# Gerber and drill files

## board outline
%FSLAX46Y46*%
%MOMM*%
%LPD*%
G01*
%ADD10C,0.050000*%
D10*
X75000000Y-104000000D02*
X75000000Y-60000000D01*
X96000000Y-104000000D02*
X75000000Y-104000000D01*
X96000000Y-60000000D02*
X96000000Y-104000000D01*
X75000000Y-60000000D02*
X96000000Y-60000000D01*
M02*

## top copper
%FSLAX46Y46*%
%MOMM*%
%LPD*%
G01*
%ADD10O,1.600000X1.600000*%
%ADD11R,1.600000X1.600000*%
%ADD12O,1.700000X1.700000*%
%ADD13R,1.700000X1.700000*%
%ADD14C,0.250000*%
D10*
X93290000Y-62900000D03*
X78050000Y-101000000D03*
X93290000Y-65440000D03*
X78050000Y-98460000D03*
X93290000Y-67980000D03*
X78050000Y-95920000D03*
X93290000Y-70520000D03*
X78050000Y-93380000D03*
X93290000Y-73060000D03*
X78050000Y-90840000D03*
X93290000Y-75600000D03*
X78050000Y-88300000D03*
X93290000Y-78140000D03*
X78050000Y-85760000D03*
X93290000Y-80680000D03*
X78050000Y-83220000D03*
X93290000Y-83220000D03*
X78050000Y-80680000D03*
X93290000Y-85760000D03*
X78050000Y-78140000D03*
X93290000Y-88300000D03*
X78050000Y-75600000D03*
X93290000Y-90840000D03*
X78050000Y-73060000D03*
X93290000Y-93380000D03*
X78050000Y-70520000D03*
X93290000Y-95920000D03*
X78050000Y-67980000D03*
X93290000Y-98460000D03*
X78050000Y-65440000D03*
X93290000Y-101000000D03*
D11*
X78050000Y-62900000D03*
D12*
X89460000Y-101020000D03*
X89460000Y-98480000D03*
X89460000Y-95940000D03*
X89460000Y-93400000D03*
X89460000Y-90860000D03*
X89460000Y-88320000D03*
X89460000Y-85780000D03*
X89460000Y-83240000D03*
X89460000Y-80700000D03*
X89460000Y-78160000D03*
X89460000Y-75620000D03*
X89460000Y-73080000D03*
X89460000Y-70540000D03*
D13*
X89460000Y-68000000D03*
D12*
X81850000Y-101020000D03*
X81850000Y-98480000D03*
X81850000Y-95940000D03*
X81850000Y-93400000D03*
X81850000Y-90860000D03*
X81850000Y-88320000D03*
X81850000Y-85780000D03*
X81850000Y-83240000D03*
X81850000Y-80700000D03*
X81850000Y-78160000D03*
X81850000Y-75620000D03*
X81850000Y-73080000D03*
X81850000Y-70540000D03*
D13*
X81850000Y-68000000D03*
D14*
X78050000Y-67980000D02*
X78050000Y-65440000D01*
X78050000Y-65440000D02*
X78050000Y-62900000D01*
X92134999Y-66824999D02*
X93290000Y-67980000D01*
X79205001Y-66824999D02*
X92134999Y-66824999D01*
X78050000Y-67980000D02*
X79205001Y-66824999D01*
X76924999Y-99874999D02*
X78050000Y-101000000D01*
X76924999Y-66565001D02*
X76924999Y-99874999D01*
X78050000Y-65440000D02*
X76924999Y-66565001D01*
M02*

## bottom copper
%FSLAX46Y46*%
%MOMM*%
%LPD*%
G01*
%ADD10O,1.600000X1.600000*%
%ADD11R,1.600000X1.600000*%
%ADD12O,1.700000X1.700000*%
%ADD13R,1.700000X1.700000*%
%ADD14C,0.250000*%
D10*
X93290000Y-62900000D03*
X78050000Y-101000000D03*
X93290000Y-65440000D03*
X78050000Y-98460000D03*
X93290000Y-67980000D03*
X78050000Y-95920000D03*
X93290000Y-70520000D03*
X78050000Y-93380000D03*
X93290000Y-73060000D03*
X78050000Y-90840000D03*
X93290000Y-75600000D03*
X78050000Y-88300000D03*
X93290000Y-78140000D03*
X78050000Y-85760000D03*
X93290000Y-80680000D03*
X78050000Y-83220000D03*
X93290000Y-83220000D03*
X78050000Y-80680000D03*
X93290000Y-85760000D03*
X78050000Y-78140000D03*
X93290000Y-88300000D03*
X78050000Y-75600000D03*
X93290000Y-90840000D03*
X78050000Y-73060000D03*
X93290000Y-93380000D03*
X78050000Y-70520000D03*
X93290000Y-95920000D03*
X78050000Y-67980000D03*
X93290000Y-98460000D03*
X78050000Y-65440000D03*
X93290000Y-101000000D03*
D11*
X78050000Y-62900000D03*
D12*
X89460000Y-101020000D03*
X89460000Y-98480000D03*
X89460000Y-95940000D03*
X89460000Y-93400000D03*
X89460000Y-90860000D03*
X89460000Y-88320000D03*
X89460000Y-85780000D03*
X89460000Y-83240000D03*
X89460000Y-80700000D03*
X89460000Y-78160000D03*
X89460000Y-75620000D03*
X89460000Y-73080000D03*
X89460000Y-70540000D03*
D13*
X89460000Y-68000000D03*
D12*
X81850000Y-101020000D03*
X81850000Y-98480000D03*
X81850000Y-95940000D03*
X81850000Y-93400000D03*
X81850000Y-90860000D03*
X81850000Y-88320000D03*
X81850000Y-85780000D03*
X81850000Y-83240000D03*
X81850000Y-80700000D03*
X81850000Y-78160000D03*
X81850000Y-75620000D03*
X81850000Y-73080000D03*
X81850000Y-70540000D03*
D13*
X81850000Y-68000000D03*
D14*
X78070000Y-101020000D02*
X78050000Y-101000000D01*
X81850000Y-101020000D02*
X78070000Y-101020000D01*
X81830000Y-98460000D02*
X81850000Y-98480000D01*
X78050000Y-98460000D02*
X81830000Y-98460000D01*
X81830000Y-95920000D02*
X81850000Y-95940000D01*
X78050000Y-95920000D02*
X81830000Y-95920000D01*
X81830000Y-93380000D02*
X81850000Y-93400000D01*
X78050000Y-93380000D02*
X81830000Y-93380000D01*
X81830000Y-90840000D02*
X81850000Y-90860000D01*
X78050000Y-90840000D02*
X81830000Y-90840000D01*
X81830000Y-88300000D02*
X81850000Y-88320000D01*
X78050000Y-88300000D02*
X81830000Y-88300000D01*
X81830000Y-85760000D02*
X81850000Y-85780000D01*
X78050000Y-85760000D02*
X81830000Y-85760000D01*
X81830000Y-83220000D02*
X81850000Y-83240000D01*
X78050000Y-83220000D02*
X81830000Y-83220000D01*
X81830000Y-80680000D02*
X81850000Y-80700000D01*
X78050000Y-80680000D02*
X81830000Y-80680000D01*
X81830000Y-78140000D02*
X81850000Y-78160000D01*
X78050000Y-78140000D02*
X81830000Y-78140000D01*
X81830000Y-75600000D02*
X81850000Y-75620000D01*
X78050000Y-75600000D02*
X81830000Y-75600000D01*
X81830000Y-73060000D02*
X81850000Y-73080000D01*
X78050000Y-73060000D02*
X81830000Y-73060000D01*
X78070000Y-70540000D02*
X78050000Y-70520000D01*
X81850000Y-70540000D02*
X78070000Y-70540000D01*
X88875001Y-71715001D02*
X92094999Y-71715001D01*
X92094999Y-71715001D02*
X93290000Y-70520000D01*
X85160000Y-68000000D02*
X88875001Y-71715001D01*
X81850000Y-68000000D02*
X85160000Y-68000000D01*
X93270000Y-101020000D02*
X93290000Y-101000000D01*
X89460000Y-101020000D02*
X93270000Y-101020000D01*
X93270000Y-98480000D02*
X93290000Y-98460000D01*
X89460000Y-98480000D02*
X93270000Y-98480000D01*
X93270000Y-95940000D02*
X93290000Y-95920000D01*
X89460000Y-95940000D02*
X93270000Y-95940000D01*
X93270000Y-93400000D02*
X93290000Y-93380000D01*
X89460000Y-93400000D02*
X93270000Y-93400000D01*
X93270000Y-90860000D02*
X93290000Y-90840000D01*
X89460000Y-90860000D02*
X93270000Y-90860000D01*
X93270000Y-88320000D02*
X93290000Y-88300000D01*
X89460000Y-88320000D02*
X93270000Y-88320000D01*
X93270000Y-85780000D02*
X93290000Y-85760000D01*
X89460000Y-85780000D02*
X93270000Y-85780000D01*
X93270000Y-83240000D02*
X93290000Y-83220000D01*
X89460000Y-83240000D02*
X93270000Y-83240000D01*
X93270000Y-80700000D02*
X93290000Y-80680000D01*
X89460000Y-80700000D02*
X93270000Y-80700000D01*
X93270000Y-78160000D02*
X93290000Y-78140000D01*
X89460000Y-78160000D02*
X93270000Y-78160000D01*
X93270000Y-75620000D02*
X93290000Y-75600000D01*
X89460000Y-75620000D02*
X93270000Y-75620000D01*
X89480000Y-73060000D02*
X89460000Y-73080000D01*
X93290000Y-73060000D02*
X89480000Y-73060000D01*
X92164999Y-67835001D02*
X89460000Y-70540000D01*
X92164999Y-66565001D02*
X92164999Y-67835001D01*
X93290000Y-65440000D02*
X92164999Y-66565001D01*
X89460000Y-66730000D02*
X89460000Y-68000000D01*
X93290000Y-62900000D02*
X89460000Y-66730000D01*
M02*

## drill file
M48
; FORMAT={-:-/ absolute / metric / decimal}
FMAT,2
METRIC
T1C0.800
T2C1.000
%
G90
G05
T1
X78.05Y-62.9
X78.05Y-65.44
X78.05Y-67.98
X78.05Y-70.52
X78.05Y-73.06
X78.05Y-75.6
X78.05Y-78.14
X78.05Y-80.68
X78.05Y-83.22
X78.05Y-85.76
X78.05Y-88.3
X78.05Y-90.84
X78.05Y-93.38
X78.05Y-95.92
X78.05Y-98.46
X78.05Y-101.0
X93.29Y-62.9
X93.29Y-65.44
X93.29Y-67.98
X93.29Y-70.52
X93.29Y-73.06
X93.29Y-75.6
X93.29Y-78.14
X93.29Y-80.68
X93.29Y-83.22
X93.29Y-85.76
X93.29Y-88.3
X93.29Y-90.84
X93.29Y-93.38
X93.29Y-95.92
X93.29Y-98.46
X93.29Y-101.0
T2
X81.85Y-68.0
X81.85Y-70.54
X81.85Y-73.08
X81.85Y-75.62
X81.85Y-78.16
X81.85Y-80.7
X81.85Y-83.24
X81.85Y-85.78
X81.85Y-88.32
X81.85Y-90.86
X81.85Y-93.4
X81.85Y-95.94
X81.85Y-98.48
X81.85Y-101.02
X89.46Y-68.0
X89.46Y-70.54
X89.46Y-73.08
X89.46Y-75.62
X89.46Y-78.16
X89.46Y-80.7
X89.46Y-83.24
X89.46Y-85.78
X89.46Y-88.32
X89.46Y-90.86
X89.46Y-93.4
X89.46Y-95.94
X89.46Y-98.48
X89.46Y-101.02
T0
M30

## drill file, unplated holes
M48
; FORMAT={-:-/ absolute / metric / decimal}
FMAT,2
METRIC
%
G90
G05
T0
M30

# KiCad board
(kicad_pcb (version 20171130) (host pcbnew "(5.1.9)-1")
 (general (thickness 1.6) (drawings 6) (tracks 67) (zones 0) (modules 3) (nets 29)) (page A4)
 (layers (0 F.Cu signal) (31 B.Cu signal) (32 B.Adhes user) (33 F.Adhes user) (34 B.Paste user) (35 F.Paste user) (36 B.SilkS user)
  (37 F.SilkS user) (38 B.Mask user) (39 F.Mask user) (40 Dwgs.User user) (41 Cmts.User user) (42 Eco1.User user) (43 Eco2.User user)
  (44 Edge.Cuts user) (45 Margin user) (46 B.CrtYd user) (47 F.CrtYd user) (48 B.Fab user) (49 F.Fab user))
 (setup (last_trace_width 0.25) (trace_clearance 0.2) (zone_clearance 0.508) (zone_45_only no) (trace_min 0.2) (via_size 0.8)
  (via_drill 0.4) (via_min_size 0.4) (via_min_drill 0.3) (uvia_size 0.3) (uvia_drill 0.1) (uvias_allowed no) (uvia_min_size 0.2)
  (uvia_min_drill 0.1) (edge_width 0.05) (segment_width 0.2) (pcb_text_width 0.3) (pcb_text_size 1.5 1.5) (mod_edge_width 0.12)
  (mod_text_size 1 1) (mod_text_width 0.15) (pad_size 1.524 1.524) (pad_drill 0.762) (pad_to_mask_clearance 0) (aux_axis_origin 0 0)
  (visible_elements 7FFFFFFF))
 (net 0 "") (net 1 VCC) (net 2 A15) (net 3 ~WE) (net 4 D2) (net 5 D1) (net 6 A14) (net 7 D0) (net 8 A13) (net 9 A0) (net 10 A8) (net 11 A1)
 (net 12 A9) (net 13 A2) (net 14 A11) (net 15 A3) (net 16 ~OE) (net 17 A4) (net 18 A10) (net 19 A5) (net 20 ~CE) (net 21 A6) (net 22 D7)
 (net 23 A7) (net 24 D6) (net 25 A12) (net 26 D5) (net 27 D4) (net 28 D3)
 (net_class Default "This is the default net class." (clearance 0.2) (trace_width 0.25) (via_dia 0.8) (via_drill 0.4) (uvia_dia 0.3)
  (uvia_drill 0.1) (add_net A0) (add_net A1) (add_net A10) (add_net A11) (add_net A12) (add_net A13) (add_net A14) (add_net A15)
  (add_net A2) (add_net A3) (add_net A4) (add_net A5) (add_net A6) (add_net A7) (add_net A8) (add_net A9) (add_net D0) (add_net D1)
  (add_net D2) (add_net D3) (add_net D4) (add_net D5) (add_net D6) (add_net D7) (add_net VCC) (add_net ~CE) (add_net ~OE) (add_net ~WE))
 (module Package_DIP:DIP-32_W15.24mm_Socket (layer F.Cu) (at 78.05 62.9)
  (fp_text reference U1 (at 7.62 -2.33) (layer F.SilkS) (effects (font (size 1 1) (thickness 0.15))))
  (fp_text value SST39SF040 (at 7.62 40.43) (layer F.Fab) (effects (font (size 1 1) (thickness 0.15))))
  (pad 32 thru_hole oval (at 15.24 0) (size 1.6 1.6) (drill 0.8) (layers *.Cu *.Mask) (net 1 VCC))
  (pad 16 thru_hole oval (at 0 38.1) (size 1.6 1.6) (drill 0.8) (layers *.Cu *.Mask) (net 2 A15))
  (pad 31 thru_hole oval (at 15.24 2.54) (size 1.6 1.6) (drill 0.8) (layers *.Cu *.Mask) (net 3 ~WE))
  (pad 15 thru_hole oval (at 0 35.56) (size 1.6 1.6) (drill 0.8) (layers *.Cu *.Mask) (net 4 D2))
  (pad 30 thru_hole oval (at 15.24 5.08) (size 1.6 1.6) (drill 0.8) (layers *.Cu *.Mask) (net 2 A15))
  (pad 14 thru_hole oval (at 0 33.02) (size 1.6 1.6) (drill 0.8) (layers *.Cu *.Mask) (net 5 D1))
  (pad 29 thru_hole oval (at 15.24 7.62) (size 1.6 1.6) (drill 0.8) (layers *.Cu *.Mask) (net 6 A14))
  (pad 13 thru_hole oval (at 0 30.48) (size 1.6 1.6) (drill 0.8) (layers *.Cu *.Mask) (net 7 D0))
  (pad 28 thru_hole oval (at 15.24 10.16) (size 1.6 1.6) (drill 0.8) (layers *.Cu *.Mask) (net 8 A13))
  (pad 12 thru_hole oval (at 0 27.94) (size 1.6 1.6) (drill 0.8) (layers *.Cu *.Mask) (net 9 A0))
  (pad 27 thru_hole oval (at 15.24 12.7) (size 1.6 1.6) (drill 0.8) (layers *.Cu *.Mask) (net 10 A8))
  (pad 11 thru_hole oval (at 0 25.4) (size 1.6 1.6) (drill 0.8) (layers *.Cu *.Mask) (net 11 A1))
  (pad 26 thru_hole oval (at 15.24 15.24) (size 1.6 1.6) (drill 0.8) (layers *.Cu *.Mask) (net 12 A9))
  (pad 10 thru_hole oval (at 0 22.86) (size 1.6 1.6) (drill 0.8) (layers *.Cu *.Mask) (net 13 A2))
  (pad 25 thru_hole oval (at 15.24 17.78) (size 1.6 1.6) (drill 0.8) (layers *.Cu *.Mask) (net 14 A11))
  (pad 9 thru_hole oval (at 0 20.32) (size 1.6 1.6) (drill 0.8) (layers *.Cu *.Mask) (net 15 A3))
  (pad 24 thru_hole oval (at 15.24 20.32) (size 1.6 1.6) (drill 0.8) (layers *.Cu *.Mask) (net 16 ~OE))
  (pad 8 thru_hole oval (at 0 17.78) (size 1.6 1.6) (drill 0.8) (layers *.Cu *.Mask) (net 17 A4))
  (pad 23 thru_hole oval (at 15.24 22.86) (size 1.6 1.6) (drill 0.8) (layers *.Cu *.Mask) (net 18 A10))
  (pad 7 thru_hole oval (at 0 15.24) (size 1.6 1.6) (drill 0.8) (layers *.Cu *.Mask) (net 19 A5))
  (pad 22 thru_hole oval (at 15.24 25.4) (size 1.6 1.6) (drill 0.8) (layers *.Cu *.Mask) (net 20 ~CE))
  (pad 6 thru_hole oval (at 0 12.7) (size 1.6 1.6) (drill 0.8) (layers *.Cu *.Mask) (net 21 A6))
  (pad 21 thru_hole oval (at 15.24 27.94) (size 1.6 1.6) (drill 0.8) (layers *.Cu *.Mask) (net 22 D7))
  (pad 5 thru_hole oval (at 0 10.16) (size 1.6 1.6) (drill 0.8) (layers *.Cu *.Mask) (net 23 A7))
  (pad 20 thru_hole oval (at 15.24 30.48) (size 1.6 1.6) (drill 0.8) (layers *.Cu *.Mask) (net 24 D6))
  (pad 4 thru_hole oval (at 0 7.62) (size 1.6 1.6) (drill 0.8) (layers *.Cu *.Mask) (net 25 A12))
  (pad 19 thru_hole oval (at 15.24 33.02) (size 1.6 1.6) (drill 0.8) (layers *.Cu *.Mask) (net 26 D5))
  (pad 3 thru_hole oval (at 0 5.08) (size 1.6 1.6) (drill 0.8) (layers *.Cu *.Mask) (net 2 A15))
  (pad 18 thru_hole oval (at 15.24 35.56) (size 1.6 1.6) (drill 0.8) (layers *.Cu *.Mask) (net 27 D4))
  (pad 2 thru_hole oval (at 0 2.54) (size 1.6 1.6) (drill 0.8) (layers *.Cu *.Mask) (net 2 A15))
  (pad 17 thru_hole oval (at 15.24 38.1) (size 1.6 1.6) (drill 0.8) (layers *.Cu *.Mask) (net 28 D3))
  (pad 1 thru_hole rect (at 0 0) (size 1.6 1.6) (drill 0.8) (layers *.Cu *.Mask) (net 2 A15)))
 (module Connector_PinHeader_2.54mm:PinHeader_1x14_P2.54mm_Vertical (layer B.Cu) (at 89.46 68 180)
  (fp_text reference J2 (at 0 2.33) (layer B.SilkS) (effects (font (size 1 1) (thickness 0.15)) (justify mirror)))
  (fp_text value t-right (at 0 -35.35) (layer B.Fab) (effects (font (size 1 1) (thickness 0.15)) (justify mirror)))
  (pad 14 thru_hole oval (at 0 -33.02 180) (size 1.7 1.7) (drill 1) (layers *.Cu *.Mask) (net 28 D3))
  (pad 13 thru_hole oval (at 0 -30.48 180) (size 1.7 1.7) (drill 1) (layers *.Cu *.Mask) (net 27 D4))
  (pad 12 thru_hole oval (at 0 -27.94 180) (size 1.7 1.7) (drill 1) (layers *.Cu *.Mask) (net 26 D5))
  (pad 11 thru_hole oval (at 0 -25.4 180) (size 1.7 1.7) (drill 1) (layers *.Cu *.Mask) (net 24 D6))
  (pad 10 thru_hole oval (at 0 -22.86 180) (size 1.7 1.7) (drill 1) (layers *.Cu *.Mask) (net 22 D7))
  (pad 9 thru_hole oval (at 0 -20.32 180) (size 1.7 1.7) (drill 1) (layers *.Cu *.Mask) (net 20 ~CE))
  (pad 8 thru_hole oval (at 0 -17.78 180) (size 1.7 1.7) (drill 1) (layers *.Cu *.Mask) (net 18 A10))
  (pad 7 thru_hole oval (at 0 -15.24 180) (size 1.7 1.7) (drill 1) (layers *.Cu *.Mask) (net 16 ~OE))
  (pad 6 thru_hole oval (at 0 -12.7 180) (size 1.7 1.7) (drill 1) (layers *.Cu *.Mask) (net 14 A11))
  (pad 5 thru_hole oval (at 0 -10.16 180) (size 1.7 1.7) (drill 1) (layers *.Cu *.Mask) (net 12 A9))
  (pad 4 thru_hole oval (at 0 -7.62 180) (size 1.7 1.7) (drill 1) (layers *.Cu *.Mask) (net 10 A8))
  (pad 3 thru_hole oval (at 0 -5.08 180) (size 1.7 1.7) (drill 1) (layers *.Cu *.Mask) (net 8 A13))
  (pad 2 thru_hole oval (at 0 -2.54 180) (size 1.7 1.7) (drill 1) (layers *.Cu *.Mask) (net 3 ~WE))
  (pad 1 thru_hole rect (at 0 0 180) (size 1.7 1.7) (drill 1) (layers *.Cu *.Mask) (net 1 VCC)))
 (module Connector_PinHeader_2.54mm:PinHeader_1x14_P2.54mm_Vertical (layer B.Cu) (at 81.85 68 180)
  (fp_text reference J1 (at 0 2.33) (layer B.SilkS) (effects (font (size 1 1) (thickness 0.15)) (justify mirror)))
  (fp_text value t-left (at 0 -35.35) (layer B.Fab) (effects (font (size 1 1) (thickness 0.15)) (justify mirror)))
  (pad 14 thru_hole oval (at 0 -33.02 180) (size 1.7 1.7) (drill 1) (layers *.Cu *.Mask) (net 2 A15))
  (pad 13 thru_hole oval (at 0 -30.48 180) (size 1.7 1.7) (drill 1) (layers *.Cu *.Mask) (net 4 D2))
  (pad 12 thru_hole oval (at 0 -27.94 180) (size 1.7 1.7) (drill 1) (layers *.Cu *.Mask) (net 5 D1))
  (pad 11 thru_hole oval (at 0 -25.4 180) (size 1.7 1.7) (drill 1) (layers *.Cu *.Mask) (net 7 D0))
  (pad 10 thru_hole oval (at 0 -22.86 180) (size 1.7 1.7) (drill 1) (layers *.Cu *.Mask) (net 9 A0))
  (pad 9 thru_hole oval (at 0 -20.32 180) (size 1.7 1.7) (drill 1) (layers *.Cu *.Mask) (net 11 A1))
  (pad 8 thru_hole oval (at 0 -17.78 180) (size 1.7 1.7) (drill 1) (layers *.Cu *.Mask) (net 13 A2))
  (pad 7 thru_hole oval (at 0 -15.24 180) (size 1.7 1.7) (drill 1) (layers *.Cu *.Mask) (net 15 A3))
  (pad 6 thru_hole oval (at 0 -12.7 180) (size 1.7 1.7) (drill 1) (layers *.Cu *.Mask) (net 17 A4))
  (pad 5 thru_hole oval (at 0 -10.16 180) (size 1.7 1.7) (drill 1) (layers *.Cu *.Mask) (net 19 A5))
  (pad 4 thru_hole oval (at 0 -7.62 180) (size 1.7 1.7) (drill 1) (layers *.Cu *.Mask) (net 21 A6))
  (pad 3 thru_hole oval (at 0 -5.08 180) (size 1.7 1.7) (drill 1) (layers *.Cu *.Mask) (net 23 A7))
  (pad 2 thru_hole oval (at 0 -2.54 180) (size 1.7 1.7) (drill 1) (layers *.Cu *.Mask) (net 25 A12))
  (pad 1 thru_hole rect (at 0 0 180) (size 1.7 1.7) (drill 1) (layers *.Cu *.Mask) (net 6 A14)))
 (gr_line (start 75 104) (end 75 60) (layer Edge.Cuts) (width 0.05))
 (gr_line (start 96 104) (end 75 104) (layer Edge.Cuts) (width 0.05))
 (gr_line (start 96 60) (end 96 104) (layer Edge.Cuts) (width 0.05))
 (gr_line (start 75 60) (end 96 60) (layer Edge.Cuts) (width 0.05))
 (segment (start 78.07 101.02) (end 78.05 101) (width 0.25) (layer B.Cu) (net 2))
 (segment (start 81.85 101.02) (end 78.07 101.02) (width 0.25) (layer B.Cu) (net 2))
 (segment (start 78.05 67.98) (end 78.05 65.44) (width 0.25) (layer F.Cu) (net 2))
 (segment (start 78.05 65.44) (end 78.05 62.9) (width 0.25) (layer F.Cu) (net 2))
 (segment (start 92.134999 66.824999) (end 93.29 67.98) (width 0.25) (layer F.Cu) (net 2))
 (segment (start 79.205001 66.824999) (end 92.134999 66.824999) (width 0.25) (layer F.Cu) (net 2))
 (segment (start 78.05 67.98) (end 79.205001 66.824999) (width 0.25) (layer F.Cu) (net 2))
 (segment (start 76.924999 99.874999) (end 78.05 101) (width 0.25) (layer F.Cu) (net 2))
 (segment (start 76.924999 66.565001) (end 76.924999 99.874999) (width 0.25) (layer F.Cu) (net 2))
 (segment (start 78.05 65.44) (end 76.924999 66.565001) (width 0.25) (layer F.Cu) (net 2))
 (segment (start 81.83 98.46) (end 81.85 98.48) (width 0.25) (layer B.Cu) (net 4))
 (segment (start 78.05 98.46) (end 81.83 98.46) (width 0.25) (layer B.Cu) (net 4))
 (segment (start 81.83 95.92) (end 81.85 95.94) (width 0.25) (layer B.Cu) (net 5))
 (segment (start 78.05 95.92) (end 81.83 95.92) (width 0.25) (layer B.Cu) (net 5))
 (segment (start 81.83 93.38) (end 81.85 93.4) (width 0.25) (layer B.Cu) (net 7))
 (segment (start 78.05 93.38) (end 81.83 93.38) (width 0.25) (layer B.Cu) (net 7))
 (segment (start 81.83 90.84) (end 81.85 90.86) (width 0.25) (layer B.Cu) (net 9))
 (segment (start 78.05 90.84) (end 81.83 90.84) (width 0.25) (layer B.Cu) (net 9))
 (segment (start 81.83 88.3) (end 81.85 88.32) (width 0.25) (layer B.Cu) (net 11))
 (segment (start 78.05 88.3) (end 81.83 88.3) (width 0.25) (layer B.Cu) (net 11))
 (segment (start 81.83 85.76) (end 81.85 85.78) (width 0.25) (layer B.Cu) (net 13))
 (segment (start 78.05 85.76) (end 81.83 85.76) (width 0.25) (layer B.Cu) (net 13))
 (segment (start 81.83 83.22) (end 81.85 83.24) (width 0.25) (layer B.Cu) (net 15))
 (segment (start 78.05 83.22) (end 81.83 83.22) (width 0.25) (layer B.Cu) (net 15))
 (segment (start 81.83 80.68) (end 81.85 80.7) (width 0.25) (layer B.Cu) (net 17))
 (segment (start 78.05 80.68) (end 81.83 80.68) (width 0.25) (layer B.Cu) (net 17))
 (segment (start 81.83 78.14) (end 81.85 78.16) (width 0.25) (layer B.Cu) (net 19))
 (segment (start 78.05 78.14) (end 81.83 78.14) (width 0.25) (layer B.Cu) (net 19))
 (segment (start 81.83 75.6) (end 81.85 75.62) (width 0.25) (layer B.Cu) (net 21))
 (segment (start 78.05 75.6) (end 81.83 75.6) (width 0.25) (layer B.Cu) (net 21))
 (segment (start 81.83 73.06) (end 81.85 73.08) (width 0.25) (layer B.Cu) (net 23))
 (segment (start 78.05 73.06) (end 81.83 73.06) (width 0.25) (layer B.Cu) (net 23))
 (segment (start 78.07 70.54) (end 78.05 70.52) (width 0.25) (layer B.Cu) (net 25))
 (segment (start 81.85 70.54) (end 78.07 70.54) (width 0.25) (layer B.Cu) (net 25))
 (segment (start 88.875001 71.715001) (end 92.094999 71.715001) (width 0.25) (layer B.Cu) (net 6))
 (segment (start 92.094999 71.715001) (end 93.29 70.52) (width 0.25) (layer B.Cu) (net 6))
 (segment (start 85.16 68) (end 88.875001 71.715001) (width 0.25) (layer B.Cu) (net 6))
 (segment (start 81.85 68) (end 85.16 68) (width 0.25) (layer B.Cu) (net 6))
 (segment (start 93.27 101.02) (end 93.29 101) (width 0.25) (layer B.Cu) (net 28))
 (segment (start 89.46 101.02) (end 93.27 101.02) (width 0.25) (layer B.Cu) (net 28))
 (segment (start 93.27 98.48) (end 93.29 98.46) (width 0.25) (layer B.Cu) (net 27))
 (segment (start 89.46 98.48) (end 93.27 98.48) (width 0.25) (layer B.Cu) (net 27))
 (segment (start 93.27 95.94) (end 93.29 95.92) (width 0.25) (layer B.Cu) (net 26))
 (segment (start 89.46 95.94) (end 93.27 95.94) (width 0.25) (layer B.Cu) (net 26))
 (segment (start 93.27 93.4) (end 93.29 93.38) (width 0.25) (layer B.Cu) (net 24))
 (segment (start 89.46 93.4) (end 93.27 93.4) (width 0.25) (layer B.Cu) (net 24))
 (segment (start 93.27 90.86) (end 93.29 90.84) (width 0.25) (layer B.Cu) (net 22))
 (segment (start 89.46 90.86) (end 93.27 90.86) (width 0.25) (layer B.Cu) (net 22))
 (segment (start 93.27 88.32) (end 93.29 88.3) (width 0.25) (layer B.Cu) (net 20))
 (segment (start 89.46 88.32) (end 93.27 88.32) (width 0.25) (layer B.Cu) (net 20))
 (segment (start 93.27 85.78) (end 93.29 85.76) (width 0.25) (layer B.Cu) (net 18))
 (segment (start 89.46 85.78) (end 93.27 85.78) (width 0.25) (layer B.Cu) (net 18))
 (segment (start 93.27 83.24) (end 93.29 83.22) (width 0.25) (layer B.Cu) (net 16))
 (segment (start 89.46 83.24) (end 93.27 83.24) (width 0.25) (layer B.Cu) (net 16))
 (segment (start 93.27 80.7) (end 93.29 80.68) (width 0.25) (layer B.Cu) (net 14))
 (segment (start 89.46 80.7) (end 93.27 80.7) (width 0.25) (layer B.Cu) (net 14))
 (segment (start 93.27 78.16) (end 93.29 78.14) (width 0.25) (layer B.Cu) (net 12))
 (segment (start 89.46 78.16) (end 93.27 78.16) (width 0.25) (layer B.Cu) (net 12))
 (segment (start 93.27 75.62) (end 93.29 75.6) (width 0.25) (layer B.Cu) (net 10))
 (segment (start 89.46 75.62) (end 93.27 75.62) (width 0.25) (layer B.Cu) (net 10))
 (segment (start 89.48 73.06) (end 89.46 73.08) (width 0.25) (layer B.Cu) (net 8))
 (segment (start 93.29 73.06) (end 89.48 73.06) (width 0.25) (layer B.Cu) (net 8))
 (segment (start 92.164999 67.835001) (end 89.46 70.54) (width 0.25) (layer B.Cu) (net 3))
 (segment (start 92.164999 66.565001) (end 92.164999 67.835001) (width 0.25) (layer B.Cu) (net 3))
 (segment (start 93.29 65.44) (end 92.164999 66.565001) (width 0.25) (layer B.Cu) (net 3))
 (segment (start 89.46 66.73) (end 89.46 68) (width 0.25) (layer B.Cu) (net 1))
 (segment (start 93.29 62.9) (end 89.46 66.73) (width 0.25) (layer B.Cu) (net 1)))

